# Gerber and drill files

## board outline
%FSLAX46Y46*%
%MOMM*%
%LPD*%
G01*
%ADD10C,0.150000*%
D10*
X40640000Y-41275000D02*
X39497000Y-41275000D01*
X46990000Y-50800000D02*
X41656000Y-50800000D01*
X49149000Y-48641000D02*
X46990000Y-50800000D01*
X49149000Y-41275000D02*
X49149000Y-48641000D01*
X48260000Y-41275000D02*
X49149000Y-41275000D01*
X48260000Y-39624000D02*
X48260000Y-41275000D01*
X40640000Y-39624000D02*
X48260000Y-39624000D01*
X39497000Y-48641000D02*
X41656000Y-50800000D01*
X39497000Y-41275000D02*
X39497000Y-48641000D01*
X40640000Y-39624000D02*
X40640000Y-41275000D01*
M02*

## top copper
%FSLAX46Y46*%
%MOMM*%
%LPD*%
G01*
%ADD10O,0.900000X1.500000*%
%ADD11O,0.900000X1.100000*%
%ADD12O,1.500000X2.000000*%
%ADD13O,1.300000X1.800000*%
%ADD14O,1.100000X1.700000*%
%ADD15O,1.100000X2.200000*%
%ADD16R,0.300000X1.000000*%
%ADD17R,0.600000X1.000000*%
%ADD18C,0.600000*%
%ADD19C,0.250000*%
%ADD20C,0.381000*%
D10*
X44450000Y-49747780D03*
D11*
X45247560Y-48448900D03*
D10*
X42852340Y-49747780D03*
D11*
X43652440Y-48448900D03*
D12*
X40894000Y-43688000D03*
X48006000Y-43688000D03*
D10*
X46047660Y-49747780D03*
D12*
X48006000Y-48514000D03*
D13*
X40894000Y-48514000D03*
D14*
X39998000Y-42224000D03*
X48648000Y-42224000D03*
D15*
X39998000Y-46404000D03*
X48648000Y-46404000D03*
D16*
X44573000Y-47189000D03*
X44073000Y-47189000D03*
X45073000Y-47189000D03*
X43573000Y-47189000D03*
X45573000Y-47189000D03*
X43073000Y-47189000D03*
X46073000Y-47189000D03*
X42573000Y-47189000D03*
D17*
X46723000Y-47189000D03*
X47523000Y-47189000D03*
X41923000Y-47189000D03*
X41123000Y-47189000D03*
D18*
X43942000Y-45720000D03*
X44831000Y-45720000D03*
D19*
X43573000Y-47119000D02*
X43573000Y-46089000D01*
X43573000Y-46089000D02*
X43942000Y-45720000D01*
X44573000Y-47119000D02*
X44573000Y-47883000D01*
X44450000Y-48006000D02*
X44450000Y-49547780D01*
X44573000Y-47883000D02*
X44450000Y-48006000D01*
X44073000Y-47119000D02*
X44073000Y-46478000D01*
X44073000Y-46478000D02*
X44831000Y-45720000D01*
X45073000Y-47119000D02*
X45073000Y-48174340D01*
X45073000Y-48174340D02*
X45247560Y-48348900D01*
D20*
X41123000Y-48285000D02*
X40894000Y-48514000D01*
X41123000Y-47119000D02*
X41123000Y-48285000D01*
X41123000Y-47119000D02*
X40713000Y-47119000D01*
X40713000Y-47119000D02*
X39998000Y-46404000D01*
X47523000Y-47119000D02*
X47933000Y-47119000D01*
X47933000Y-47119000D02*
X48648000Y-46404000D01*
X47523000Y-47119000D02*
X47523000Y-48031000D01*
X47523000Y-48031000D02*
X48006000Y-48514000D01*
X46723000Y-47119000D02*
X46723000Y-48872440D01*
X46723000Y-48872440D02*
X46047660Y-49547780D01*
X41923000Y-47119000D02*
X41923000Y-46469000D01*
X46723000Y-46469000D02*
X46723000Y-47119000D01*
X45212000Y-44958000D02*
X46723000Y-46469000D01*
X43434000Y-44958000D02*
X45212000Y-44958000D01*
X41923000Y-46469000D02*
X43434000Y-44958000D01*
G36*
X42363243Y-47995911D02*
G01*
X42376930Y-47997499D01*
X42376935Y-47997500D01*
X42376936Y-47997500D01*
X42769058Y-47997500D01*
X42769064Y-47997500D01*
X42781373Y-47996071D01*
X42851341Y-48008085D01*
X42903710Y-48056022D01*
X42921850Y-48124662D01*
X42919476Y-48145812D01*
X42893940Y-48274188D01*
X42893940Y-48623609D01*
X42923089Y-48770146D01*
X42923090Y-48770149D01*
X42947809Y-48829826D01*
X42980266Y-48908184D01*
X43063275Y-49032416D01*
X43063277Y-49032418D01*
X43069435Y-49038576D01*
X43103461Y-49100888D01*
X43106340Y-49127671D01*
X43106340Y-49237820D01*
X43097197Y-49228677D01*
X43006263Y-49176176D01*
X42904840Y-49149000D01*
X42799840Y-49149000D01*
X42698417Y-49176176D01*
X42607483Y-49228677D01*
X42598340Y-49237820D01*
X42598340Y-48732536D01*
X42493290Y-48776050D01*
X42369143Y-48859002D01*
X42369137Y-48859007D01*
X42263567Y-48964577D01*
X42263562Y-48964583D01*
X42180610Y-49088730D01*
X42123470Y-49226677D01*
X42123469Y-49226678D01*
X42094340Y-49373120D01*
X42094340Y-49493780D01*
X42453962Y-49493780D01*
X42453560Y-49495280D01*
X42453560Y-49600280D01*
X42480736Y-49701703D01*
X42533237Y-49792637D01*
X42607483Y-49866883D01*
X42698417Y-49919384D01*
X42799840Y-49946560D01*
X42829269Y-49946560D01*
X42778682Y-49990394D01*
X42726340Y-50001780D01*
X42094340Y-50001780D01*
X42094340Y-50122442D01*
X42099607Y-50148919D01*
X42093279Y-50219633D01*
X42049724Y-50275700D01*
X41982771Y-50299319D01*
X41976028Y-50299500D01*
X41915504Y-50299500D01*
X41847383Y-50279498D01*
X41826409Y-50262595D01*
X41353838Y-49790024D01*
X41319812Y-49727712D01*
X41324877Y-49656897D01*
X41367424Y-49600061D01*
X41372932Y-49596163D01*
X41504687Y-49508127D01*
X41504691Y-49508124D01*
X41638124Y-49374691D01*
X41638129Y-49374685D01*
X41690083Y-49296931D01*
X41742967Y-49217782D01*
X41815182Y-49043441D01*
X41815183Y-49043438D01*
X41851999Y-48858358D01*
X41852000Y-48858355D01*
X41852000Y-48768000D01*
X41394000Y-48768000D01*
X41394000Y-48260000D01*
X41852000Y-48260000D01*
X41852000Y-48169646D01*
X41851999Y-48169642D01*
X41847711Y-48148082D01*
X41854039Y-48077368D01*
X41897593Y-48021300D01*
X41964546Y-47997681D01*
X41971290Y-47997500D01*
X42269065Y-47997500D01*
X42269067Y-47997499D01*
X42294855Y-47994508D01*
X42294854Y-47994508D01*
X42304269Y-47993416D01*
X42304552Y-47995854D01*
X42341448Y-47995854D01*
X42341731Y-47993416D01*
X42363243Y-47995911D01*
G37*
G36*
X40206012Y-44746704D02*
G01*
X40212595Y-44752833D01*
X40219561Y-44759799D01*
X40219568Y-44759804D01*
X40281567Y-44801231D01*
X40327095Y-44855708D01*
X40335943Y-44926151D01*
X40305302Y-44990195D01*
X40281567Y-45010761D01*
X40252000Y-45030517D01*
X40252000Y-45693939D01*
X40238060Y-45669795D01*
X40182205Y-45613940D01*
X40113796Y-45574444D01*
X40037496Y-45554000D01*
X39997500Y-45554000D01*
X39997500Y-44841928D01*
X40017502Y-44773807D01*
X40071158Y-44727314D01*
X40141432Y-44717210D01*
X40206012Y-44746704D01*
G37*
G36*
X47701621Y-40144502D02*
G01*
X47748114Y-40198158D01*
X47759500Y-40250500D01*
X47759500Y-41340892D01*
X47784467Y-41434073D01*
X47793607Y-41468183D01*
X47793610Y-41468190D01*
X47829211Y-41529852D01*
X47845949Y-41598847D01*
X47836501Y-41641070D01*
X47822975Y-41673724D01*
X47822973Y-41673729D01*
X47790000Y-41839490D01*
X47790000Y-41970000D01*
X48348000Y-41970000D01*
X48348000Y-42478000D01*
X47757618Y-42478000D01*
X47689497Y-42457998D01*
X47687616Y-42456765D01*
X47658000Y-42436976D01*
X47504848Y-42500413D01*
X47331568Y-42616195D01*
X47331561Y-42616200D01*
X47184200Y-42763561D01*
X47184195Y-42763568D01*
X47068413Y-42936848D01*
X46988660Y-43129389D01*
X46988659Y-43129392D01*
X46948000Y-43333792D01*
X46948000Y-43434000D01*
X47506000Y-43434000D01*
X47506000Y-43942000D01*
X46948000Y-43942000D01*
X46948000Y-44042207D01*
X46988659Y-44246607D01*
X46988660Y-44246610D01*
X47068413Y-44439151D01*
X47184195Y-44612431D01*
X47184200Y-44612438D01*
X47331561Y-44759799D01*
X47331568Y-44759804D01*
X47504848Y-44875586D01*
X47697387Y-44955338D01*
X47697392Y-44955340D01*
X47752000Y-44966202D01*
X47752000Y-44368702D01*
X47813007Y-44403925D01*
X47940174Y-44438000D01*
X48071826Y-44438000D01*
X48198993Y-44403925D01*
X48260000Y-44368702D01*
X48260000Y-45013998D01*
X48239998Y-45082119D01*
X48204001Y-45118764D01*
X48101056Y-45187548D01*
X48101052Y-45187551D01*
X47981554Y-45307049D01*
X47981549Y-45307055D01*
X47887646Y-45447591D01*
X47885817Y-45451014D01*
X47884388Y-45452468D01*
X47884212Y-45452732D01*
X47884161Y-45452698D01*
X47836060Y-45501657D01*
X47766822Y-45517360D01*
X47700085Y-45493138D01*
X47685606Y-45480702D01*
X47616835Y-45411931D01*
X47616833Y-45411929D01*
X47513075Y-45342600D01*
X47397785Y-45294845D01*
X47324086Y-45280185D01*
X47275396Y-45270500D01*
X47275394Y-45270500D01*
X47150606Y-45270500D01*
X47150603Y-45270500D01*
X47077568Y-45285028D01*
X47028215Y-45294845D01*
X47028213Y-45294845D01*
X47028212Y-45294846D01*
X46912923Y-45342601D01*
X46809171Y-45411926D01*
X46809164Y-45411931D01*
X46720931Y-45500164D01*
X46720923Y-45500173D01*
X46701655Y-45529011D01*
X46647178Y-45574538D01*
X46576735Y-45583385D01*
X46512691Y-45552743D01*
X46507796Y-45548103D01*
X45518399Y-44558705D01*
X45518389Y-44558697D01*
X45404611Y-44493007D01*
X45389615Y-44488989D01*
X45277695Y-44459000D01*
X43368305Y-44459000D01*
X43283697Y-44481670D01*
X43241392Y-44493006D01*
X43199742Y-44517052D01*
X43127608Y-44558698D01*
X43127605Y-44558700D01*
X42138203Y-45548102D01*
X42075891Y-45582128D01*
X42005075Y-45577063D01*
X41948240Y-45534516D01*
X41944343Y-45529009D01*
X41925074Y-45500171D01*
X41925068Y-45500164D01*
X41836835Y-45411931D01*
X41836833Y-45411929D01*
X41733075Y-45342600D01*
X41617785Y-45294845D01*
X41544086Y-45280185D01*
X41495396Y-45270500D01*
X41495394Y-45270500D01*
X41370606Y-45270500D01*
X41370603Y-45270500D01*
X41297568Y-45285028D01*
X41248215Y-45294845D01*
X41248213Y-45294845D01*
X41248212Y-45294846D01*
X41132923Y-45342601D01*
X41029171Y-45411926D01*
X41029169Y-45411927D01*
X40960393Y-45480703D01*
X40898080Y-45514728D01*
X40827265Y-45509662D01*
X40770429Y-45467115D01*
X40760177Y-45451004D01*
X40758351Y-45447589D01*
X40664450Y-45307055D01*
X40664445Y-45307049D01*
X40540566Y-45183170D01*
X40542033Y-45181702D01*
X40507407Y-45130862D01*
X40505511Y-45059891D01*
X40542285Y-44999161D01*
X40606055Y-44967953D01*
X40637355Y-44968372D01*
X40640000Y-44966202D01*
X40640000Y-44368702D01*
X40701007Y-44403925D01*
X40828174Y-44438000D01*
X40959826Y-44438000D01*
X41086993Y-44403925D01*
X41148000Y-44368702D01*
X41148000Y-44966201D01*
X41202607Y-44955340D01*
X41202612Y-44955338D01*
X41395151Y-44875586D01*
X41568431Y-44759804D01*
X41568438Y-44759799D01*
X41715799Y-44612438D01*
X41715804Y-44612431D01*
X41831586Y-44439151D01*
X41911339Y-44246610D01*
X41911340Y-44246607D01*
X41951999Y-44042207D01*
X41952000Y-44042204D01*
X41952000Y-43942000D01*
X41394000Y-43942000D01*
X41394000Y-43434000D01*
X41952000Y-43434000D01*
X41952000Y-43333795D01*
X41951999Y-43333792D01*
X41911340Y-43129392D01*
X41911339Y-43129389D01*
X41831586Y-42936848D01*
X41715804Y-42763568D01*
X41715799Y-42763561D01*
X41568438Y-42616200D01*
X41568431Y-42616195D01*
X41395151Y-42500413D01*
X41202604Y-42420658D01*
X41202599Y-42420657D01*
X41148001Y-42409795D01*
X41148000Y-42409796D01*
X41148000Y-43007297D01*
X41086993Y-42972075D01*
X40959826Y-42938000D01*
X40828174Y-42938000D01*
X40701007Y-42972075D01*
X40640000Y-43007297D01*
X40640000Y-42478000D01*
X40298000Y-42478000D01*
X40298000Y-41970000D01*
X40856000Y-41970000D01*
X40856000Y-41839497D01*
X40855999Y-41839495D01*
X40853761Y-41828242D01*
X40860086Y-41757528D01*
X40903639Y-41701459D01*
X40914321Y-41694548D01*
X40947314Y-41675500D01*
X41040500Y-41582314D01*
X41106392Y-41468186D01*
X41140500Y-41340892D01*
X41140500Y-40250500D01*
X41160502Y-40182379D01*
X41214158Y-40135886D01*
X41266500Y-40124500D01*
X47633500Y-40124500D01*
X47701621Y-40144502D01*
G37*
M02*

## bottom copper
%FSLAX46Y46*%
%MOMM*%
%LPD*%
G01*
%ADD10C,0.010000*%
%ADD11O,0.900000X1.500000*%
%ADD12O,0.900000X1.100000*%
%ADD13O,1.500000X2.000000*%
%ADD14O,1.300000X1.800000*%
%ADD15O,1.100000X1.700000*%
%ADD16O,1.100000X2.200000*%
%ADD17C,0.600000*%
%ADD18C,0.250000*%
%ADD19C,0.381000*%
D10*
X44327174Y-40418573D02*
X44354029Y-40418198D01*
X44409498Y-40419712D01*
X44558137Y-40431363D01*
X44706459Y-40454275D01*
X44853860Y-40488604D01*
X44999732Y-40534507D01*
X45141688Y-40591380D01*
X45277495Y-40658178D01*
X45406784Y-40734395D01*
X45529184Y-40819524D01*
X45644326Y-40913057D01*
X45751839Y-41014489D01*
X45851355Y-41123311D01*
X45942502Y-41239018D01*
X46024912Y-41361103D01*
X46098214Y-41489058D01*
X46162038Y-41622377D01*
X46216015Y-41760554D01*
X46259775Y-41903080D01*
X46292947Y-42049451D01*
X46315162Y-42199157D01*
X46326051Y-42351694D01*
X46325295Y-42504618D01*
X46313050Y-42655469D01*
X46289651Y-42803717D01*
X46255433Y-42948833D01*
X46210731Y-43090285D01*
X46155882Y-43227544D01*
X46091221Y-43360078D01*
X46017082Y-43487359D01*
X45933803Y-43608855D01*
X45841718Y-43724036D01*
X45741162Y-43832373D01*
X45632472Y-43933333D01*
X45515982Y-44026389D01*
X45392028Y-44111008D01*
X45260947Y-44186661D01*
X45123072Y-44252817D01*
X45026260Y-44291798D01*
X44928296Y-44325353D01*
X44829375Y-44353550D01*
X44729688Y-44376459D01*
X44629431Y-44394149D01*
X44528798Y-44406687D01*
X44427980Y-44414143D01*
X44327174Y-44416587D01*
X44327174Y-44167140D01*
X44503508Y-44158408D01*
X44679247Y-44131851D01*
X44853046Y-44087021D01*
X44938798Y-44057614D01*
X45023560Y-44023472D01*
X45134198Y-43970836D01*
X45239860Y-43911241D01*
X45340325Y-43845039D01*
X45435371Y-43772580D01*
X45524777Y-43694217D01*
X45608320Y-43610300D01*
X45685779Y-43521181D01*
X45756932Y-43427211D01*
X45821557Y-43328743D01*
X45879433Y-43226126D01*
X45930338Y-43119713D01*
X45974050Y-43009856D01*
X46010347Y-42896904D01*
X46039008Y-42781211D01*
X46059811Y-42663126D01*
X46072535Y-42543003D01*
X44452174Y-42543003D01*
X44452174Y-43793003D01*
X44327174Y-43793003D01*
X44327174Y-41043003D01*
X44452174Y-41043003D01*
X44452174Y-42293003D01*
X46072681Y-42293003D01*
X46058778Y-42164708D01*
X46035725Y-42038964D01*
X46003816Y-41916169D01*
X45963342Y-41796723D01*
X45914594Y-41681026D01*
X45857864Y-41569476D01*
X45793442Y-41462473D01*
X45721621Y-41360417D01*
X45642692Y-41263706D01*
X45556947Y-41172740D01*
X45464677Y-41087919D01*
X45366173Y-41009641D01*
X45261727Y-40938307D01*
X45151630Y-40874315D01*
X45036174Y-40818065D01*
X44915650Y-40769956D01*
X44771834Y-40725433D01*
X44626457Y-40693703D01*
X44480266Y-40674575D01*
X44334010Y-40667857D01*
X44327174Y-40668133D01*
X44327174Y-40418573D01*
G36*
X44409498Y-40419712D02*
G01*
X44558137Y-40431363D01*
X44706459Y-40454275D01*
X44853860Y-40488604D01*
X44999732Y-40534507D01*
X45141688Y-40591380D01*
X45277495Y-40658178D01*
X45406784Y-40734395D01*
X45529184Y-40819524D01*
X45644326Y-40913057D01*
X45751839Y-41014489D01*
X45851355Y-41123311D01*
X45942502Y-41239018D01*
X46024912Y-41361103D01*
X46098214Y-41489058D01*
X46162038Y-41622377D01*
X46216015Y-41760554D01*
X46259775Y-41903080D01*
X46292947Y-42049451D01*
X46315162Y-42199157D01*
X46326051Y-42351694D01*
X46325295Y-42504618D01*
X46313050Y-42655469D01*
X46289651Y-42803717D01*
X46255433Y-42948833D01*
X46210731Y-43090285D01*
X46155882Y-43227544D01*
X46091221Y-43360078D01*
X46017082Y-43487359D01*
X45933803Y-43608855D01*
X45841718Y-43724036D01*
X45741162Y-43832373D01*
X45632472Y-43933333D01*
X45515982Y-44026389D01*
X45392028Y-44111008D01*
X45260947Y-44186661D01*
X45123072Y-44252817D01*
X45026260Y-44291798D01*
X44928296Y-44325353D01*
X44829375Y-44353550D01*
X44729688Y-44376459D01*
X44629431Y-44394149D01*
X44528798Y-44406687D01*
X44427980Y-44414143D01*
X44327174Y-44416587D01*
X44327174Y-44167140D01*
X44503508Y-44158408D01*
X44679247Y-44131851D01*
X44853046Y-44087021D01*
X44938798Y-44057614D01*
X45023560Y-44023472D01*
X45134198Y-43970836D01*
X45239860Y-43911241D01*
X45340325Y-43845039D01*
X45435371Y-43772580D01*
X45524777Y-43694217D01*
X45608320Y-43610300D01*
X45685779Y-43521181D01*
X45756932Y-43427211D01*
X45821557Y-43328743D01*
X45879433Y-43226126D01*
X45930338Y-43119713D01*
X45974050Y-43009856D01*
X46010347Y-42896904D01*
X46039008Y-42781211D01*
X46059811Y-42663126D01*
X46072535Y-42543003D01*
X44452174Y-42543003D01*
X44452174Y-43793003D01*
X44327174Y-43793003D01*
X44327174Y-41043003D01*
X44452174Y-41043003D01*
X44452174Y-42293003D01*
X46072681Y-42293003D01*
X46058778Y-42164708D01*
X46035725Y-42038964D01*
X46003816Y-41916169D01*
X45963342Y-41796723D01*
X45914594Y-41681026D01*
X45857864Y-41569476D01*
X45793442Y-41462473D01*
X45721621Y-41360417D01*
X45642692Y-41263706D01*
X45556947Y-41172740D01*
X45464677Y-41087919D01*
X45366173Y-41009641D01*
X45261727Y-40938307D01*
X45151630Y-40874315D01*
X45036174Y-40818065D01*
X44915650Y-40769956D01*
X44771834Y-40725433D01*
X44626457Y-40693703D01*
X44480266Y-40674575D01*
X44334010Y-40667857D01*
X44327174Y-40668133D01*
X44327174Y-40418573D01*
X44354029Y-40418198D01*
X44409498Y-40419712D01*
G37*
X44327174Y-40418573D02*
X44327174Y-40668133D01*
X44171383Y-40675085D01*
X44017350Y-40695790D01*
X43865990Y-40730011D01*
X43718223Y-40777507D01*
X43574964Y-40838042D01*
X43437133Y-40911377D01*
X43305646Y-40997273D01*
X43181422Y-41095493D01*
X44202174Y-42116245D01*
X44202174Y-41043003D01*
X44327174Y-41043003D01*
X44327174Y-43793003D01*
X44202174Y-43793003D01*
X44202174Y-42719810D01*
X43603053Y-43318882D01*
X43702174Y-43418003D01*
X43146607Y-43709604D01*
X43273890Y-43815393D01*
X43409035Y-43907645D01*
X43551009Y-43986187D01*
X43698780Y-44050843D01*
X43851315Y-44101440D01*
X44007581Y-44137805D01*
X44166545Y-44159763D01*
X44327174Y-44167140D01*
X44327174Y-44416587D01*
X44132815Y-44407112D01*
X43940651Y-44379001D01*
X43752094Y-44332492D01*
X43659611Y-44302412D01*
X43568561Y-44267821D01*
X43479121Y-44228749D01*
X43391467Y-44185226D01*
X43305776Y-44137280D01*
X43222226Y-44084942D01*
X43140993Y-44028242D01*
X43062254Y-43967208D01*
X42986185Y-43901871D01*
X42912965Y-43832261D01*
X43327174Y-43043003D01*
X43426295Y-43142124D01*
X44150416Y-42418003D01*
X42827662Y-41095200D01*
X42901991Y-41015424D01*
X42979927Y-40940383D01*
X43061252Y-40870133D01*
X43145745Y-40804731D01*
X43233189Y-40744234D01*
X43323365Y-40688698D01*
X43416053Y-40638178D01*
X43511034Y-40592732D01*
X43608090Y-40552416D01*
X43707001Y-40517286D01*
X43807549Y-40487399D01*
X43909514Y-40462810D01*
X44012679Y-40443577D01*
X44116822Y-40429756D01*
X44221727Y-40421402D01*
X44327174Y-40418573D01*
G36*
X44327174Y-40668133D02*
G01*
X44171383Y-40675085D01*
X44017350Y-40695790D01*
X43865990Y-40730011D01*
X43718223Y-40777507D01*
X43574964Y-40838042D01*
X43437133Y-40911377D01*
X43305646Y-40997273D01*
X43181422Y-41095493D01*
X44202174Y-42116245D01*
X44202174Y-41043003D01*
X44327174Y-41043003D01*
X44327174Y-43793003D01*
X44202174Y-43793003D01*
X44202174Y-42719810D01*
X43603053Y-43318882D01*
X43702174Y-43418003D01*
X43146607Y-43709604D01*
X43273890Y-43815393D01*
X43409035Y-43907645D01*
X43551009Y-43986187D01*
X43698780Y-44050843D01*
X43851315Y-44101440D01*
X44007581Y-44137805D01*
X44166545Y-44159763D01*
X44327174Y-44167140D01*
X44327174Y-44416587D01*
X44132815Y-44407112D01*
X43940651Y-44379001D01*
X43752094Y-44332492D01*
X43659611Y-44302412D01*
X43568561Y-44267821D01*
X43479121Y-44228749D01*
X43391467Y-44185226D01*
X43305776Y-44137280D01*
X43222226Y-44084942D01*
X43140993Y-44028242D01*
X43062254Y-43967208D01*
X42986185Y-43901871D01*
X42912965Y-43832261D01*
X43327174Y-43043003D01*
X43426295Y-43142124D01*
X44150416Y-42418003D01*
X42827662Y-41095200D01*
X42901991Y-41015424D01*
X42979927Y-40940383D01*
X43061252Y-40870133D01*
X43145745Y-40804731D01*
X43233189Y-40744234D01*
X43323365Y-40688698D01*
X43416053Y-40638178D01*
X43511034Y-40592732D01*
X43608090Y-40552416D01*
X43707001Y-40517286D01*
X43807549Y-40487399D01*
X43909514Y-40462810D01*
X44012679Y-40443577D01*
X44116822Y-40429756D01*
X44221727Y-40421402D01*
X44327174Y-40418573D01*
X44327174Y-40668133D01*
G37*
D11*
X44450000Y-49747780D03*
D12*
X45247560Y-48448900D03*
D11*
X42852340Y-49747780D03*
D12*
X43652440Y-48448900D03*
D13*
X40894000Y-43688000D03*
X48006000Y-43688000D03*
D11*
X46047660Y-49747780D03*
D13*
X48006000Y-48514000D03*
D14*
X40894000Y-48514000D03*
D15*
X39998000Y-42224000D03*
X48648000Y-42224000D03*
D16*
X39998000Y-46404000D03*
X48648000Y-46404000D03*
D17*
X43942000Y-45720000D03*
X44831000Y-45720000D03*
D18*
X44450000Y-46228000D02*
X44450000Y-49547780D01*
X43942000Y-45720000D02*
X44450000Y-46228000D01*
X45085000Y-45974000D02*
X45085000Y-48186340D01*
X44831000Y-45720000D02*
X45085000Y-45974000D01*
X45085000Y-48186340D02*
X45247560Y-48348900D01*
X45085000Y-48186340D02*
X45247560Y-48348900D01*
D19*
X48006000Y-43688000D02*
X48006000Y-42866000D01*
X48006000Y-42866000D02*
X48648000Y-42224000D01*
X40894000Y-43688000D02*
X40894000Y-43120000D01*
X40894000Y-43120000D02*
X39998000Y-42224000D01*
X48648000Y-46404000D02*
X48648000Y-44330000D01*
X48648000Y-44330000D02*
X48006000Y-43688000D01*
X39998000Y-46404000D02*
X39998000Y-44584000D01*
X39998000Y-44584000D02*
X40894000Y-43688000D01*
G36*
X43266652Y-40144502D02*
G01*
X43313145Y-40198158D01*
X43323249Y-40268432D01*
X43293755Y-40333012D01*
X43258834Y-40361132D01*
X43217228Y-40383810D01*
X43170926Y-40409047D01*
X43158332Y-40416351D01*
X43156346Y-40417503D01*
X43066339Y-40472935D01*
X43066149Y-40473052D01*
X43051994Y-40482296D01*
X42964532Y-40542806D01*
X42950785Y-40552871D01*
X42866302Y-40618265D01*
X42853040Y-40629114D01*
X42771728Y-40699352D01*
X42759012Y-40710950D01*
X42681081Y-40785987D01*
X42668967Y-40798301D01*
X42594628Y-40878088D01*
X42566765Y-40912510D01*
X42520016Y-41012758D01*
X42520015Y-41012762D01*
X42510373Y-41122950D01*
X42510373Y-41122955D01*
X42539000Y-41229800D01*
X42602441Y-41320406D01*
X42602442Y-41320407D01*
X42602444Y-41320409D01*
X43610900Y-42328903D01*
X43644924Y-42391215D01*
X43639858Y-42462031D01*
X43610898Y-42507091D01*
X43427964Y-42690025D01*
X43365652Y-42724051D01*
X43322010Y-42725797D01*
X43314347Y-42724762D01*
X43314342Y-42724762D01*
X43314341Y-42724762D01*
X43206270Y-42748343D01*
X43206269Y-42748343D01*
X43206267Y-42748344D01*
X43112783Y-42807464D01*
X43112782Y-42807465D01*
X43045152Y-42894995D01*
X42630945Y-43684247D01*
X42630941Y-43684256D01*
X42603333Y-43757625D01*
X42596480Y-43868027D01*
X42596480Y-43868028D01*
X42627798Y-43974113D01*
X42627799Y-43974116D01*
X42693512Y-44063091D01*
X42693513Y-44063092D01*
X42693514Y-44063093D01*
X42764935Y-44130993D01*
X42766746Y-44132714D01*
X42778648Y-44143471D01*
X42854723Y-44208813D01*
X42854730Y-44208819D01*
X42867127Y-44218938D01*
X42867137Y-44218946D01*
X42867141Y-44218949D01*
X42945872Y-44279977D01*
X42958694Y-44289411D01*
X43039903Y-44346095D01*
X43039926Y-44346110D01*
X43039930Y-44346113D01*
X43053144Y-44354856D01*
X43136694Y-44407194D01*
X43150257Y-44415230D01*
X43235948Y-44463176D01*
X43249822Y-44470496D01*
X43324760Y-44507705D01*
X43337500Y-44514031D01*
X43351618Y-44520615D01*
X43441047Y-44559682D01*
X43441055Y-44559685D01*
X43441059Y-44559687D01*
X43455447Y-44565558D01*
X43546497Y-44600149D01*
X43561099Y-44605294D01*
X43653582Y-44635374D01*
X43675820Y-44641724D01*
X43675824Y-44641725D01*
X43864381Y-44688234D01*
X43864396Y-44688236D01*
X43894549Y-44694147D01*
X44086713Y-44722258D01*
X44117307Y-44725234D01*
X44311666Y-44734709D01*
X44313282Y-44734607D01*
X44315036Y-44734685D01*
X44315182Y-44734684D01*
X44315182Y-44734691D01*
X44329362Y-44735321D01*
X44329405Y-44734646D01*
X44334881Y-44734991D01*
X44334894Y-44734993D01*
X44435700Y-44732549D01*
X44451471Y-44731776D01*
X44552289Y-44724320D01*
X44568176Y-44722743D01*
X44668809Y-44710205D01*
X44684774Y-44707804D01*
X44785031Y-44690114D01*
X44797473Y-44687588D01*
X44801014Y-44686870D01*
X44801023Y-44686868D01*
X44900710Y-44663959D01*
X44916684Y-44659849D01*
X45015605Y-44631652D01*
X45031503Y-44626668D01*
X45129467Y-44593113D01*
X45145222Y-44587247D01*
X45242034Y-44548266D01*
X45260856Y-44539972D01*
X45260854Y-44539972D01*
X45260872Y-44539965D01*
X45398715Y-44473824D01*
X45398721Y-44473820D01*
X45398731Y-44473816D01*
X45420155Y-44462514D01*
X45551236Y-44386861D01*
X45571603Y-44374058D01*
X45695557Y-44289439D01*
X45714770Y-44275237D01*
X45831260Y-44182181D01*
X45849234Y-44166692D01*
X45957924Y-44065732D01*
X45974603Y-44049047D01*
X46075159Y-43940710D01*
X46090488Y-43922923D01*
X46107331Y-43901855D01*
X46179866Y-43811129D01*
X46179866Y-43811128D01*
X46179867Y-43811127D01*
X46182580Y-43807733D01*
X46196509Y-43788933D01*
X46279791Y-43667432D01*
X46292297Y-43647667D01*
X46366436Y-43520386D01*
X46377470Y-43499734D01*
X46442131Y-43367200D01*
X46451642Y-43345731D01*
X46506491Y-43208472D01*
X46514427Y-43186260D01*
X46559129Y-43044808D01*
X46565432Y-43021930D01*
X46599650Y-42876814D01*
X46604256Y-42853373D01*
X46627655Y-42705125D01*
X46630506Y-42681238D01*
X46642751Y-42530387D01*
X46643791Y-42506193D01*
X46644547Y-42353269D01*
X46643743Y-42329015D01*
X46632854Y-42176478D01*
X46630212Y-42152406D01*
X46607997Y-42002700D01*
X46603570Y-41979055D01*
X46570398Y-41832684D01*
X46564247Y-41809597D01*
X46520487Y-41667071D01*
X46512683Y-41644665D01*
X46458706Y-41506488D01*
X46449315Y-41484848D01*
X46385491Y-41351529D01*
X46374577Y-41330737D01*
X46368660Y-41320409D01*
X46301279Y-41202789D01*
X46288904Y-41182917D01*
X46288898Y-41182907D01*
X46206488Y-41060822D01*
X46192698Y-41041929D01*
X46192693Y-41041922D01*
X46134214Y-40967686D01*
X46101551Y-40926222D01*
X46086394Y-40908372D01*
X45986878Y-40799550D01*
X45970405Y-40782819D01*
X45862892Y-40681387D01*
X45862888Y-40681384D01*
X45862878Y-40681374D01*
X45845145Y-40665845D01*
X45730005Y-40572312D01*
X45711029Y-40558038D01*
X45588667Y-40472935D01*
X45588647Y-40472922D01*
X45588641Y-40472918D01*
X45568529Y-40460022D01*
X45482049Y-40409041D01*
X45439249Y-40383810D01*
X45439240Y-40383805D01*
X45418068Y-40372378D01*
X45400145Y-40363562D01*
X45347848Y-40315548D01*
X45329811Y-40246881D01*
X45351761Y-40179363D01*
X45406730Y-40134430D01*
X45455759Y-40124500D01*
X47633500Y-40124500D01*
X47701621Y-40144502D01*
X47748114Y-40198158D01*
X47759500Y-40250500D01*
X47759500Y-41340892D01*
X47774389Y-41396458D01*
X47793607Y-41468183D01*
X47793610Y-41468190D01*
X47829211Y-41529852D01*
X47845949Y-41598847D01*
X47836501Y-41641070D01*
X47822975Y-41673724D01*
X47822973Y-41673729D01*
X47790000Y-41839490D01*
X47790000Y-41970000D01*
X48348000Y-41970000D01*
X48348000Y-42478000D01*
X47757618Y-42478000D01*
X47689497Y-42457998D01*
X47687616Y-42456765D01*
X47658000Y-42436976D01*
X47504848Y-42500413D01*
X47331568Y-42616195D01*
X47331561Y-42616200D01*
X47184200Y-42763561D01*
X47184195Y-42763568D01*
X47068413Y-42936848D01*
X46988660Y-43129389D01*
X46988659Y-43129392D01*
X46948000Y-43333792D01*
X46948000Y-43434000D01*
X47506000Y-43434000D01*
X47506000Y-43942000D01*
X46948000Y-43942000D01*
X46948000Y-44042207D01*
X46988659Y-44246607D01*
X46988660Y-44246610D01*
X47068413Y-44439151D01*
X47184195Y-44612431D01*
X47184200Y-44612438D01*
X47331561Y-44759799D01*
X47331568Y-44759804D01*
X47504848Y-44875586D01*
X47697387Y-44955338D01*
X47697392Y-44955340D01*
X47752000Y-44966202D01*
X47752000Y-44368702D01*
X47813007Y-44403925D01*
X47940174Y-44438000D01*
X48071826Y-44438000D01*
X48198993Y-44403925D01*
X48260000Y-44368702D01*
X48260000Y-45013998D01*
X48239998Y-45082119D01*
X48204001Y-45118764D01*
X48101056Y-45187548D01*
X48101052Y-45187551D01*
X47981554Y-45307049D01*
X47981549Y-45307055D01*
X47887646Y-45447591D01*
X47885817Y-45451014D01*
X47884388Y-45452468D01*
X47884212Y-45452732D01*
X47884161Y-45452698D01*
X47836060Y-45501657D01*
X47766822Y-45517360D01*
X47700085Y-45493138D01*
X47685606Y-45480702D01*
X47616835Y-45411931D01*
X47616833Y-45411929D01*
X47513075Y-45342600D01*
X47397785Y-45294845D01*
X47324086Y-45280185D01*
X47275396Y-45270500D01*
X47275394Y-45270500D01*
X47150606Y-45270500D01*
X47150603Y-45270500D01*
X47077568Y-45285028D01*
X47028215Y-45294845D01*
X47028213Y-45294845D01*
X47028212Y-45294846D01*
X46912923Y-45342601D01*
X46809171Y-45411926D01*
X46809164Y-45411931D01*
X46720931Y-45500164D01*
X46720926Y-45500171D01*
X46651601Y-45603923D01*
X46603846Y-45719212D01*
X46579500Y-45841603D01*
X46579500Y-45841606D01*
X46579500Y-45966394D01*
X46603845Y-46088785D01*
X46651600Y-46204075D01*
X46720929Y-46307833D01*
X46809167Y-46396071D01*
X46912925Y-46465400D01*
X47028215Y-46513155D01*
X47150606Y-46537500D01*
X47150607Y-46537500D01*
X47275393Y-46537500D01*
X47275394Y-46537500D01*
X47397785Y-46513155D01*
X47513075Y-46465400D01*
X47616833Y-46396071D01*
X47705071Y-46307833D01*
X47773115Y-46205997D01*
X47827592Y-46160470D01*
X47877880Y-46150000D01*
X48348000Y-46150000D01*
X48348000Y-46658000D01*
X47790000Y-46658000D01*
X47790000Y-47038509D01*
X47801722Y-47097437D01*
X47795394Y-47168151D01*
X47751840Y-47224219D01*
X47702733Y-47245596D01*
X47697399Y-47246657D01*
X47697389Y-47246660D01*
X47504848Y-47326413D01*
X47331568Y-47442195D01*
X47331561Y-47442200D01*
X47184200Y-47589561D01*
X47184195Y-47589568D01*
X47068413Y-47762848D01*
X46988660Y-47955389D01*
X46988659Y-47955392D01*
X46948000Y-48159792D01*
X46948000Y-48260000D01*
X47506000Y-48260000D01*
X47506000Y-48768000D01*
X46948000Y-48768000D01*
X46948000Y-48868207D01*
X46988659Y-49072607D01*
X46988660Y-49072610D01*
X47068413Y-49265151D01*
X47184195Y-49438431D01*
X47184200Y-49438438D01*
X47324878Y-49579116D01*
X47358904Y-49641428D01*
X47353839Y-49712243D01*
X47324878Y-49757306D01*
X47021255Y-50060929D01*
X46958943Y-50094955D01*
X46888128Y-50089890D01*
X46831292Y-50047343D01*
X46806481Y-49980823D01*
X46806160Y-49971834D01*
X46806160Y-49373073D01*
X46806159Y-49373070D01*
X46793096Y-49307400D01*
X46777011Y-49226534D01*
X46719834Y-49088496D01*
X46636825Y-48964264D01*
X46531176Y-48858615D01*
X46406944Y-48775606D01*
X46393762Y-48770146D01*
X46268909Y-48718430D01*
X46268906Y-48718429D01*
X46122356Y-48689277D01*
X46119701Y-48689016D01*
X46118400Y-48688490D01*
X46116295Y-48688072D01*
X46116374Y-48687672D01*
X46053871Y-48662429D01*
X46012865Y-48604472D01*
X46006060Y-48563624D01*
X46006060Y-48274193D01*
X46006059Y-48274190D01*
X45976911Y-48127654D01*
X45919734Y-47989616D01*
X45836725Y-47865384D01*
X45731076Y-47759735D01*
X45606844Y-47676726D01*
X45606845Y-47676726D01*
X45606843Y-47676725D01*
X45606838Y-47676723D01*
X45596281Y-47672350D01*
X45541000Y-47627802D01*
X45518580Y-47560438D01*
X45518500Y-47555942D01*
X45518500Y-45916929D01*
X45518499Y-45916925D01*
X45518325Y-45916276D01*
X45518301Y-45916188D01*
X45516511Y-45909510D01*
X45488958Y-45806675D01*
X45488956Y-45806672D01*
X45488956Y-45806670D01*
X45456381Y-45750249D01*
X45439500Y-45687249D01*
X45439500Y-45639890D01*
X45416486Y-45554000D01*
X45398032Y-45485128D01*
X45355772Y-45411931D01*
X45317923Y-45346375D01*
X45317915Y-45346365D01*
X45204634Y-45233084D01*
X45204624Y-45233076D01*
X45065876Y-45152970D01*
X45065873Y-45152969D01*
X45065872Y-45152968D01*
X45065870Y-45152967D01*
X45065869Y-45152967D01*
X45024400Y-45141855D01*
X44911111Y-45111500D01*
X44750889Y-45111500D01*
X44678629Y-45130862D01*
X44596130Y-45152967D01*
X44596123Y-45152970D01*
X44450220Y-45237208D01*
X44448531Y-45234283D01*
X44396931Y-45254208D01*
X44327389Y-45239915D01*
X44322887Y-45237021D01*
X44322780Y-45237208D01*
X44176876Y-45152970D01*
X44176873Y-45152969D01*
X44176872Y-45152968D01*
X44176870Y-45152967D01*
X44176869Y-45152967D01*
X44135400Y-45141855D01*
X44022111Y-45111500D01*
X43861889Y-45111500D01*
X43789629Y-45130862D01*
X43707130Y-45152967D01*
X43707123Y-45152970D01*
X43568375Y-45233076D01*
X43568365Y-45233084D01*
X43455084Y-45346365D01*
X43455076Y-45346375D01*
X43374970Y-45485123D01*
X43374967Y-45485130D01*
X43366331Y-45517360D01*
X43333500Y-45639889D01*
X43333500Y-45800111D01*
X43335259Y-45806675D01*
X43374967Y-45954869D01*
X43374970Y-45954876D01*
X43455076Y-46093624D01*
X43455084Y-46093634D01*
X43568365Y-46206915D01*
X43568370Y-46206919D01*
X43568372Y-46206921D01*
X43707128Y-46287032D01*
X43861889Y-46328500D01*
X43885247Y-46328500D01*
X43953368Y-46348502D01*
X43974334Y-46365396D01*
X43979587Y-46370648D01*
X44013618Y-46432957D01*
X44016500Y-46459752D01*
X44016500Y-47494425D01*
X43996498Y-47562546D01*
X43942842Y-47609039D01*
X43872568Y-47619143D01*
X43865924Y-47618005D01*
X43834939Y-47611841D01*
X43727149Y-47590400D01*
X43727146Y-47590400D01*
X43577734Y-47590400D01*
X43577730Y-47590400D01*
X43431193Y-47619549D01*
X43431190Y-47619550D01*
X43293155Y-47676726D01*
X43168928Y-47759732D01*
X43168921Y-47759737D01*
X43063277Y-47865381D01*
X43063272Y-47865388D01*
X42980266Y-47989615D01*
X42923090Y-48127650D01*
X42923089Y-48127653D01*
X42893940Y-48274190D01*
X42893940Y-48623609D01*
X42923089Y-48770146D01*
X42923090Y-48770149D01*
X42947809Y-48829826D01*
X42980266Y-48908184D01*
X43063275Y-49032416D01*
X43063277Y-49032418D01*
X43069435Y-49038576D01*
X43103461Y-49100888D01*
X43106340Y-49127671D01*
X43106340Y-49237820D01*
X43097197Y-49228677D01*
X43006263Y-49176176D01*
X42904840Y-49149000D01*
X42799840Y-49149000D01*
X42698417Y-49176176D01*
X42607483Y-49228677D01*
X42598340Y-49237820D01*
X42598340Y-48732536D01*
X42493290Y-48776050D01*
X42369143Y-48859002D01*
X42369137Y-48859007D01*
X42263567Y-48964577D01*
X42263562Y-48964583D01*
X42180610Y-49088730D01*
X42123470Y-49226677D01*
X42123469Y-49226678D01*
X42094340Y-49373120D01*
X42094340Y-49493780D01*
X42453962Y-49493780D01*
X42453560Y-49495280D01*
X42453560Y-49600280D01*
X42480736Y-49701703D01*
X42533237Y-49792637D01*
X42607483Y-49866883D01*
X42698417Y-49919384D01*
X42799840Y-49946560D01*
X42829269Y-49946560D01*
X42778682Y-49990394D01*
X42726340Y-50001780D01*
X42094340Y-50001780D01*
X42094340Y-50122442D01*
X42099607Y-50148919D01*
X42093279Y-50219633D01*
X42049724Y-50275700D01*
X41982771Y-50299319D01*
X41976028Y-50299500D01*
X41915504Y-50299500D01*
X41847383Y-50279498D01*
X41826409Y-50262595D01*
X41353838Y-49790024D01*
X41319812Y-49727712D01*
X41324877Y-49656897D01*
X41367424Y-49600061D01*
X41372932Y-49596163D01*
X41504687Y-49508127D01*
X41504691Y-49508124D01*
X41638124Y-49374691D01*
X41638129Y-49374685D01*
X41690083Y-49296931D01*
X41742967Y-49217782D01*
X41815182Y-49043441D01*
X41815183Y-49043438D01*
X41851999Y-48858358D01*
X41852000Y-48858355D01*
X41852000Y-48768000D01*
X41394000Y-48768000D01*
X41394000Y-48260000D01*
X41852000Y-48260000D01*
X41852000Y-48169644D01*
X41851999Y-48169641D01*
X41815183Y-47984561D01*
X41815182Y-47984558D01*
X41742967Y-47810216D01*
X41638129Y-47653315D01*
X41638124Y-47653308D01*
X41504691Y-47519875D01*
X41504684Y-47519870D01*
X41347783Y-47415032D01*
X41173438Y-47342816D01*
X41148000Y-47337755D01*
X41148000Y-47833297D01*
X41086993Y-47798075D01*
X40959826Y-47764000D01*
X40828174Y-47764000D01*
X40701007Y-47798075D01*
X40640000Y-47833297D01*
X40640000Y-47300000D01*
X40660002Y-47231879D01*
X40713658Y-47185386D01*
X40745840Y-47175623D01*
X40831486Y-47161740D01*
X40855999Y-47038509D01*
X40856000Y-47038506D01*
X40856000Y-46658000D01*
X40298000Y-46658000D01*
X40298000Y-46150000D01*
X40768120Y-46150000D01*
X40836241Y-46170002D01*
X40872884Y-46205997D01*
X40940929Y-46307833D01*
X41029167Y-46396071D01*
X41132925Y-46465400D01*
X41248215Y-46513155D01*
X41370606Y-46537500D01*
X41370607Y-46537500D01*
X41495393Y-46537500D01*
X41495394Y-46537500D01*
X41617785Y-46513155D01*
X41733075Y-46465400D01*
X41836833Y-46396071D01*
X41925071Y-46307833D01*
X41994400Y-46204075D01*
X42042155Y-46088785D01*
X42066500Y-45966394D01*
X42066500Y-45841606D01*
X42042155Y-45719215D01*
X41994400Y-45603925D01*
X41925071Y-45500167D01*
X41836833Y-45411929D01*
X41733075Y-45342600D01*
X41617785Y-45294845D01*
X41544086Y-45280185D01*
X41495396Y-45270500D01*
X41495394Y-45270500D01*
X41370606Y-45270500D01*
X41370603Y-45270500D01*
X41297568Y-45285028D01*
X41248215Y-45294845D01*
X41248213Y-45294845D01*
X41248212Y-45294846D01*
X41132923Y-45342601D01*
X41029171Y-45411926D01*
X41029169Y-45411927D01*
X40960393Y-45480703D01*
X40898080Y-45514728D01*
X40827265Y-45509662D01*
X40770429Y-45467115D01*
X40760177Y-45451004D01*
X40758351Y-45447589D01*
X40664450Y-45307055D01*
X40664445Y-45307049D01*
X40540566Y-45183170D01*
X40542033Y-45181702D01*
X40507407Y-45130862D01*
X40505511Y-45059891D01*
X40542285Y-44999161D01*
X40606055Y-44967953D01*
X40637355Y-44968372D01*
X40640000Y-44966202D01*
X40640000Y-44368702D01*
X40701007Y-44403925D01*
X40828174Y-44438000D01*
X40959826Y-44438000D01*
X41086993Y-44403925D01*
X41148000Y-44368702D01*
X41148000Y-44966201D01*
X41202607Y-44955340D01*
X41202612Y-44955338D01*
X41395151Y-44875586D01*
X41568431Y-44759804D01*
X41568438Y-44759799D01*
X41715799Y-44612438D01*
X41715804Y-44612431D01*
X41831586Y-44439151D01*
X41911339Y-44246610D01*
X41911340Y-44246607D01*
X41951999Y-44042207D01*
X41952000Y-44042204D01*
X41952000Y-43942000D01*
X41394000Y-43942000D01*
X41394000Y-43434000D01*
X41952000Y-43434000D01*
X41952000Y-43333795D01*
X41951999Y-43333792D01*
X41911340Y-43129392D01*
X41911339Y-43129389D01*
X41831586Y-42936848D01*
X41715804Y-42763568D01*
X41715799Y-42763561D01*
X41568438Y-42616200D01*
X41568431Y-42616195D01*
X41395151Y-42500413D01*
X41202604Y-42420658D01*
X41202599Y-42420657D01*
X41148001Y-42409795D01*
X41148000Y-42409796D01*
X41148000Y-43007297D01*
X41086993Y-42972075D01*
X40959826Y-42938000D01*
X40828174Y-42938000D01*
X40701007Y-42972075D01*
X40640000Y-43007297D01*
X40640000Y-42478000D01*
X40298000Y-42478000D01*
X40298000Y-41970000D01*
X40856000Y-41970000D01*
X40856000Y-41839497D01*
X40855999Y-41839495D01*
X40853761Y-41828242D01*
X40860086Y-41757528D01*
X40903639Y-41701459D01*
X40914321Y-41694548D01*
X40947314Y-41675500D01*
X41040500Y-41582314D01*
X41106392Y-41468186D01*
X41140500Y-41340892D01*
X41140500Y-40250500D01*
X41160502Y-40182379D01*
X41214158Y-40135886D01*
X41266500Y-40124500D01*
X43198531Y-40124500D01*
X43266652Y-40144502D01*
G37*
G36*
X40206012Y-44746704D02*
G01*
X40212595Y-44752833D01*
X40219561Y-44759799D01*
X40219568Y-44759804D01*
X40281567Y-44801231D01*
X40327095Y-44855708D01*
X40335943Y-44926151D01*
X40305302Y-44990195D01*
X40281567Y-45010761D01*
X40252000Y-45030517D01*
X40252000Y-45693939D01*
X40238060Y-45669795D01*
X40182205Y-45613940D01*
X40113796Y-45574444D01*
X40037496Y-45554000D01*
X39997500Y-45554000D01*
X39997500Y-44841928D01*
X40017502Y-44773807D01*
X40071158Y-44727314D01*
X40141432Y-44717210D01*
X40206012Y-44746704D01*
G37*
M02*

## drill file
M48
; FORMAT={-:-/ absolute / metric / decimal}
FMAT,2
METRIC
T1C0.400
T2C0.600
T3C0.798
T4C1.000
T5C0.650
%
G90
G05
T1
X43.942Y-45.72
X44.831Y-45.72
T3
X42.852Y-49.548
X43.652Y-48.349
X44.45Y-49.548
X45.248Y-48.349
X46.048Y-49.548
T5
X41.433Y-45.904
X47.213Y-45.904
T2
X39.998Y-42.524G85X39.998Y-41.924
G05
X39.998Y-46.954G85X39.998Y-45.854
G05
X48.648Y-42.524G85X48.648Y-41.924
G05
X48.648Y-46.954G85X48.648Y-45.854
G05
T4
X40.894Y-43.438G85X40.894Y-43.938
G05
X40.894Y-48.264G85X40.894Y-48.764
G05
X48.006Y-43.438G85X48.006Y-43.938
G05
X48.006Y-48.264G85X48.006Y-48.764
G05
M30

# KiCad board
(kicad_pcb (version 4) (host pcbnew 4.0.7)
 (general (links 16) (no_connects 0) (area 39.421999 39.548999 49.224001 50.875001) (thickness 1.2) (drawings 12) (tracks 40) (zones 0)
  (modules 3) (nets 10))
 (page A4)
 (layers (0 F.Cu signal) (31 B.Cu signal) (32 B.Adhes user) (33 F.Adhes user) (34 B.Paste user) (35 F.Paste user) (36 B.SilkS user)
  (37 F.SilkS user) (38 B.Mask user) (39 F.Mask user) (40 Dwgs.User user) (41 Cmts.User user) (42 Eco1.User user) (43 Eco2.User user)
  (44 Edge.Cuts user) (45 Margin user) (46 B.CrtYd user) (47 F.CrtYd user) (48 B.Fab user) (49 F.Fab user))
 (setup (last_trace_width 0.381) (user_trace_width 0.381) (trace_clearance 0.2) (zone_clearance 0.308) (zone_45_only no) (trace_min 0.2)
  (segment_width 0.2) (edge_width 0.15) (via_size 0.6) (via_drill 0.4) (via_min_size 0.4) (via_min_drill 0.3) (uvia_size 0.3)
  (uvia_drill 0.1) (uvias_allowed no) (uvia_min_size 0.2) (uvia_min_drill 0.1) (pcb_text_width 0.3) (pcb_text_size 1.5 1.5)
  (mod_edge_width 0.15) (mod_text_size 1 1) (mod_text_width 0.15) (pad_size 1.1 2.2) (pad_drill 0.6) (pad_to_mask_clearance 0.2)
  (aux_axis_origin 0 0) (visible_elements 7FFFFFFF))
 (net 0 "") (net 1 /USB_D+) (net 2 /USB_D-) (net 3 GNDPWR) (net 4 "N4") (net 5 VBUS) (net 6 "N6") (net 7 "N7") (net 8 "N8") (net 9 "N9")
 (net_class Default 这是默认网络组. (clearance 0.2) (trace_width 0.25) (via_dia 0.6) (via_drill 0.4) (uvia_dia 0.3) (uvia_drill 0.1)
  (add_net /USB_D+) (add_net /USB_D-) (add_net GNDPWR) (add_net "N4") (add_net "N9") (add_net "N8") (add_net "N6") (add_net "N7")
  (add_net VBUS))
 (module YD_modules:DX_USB (layer F.Cu) (at 44.45 44.45 270)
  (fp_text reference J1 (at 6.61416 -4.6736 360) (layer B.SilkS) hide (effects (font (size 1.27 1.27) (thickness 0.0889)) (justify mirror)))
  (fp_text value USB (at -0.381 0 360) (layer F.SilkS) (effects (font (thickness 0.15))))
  (pad 3 thru_hole oval (at 5.09778 0 270) (size 1.5 0.9) (drill 0.79756 (offset 0.2 0)) (layers *.Cu *.Paste *.Mask) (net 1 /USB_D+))
  (pad 2 thru_hole oval (at 3.8989 -0.79756 270) (size 1.1 0.9) (drill 0.79756 (offset 0.1 0)) (layers *.Cu *.Paste *.Mask) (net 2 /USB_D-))
  (pad 5 thru_hole oval (at 5.09778 1.59766 270) (size 1.5 0.9) (drill 0.79756 (offset 0.2 0)) (layers *.Cu *.Paste *.Mask) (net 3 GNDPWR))
  (pad 4 thru_hole oval (at 3.8989 0.79756 270) (size 1.1 0.9) (drill 0.79756 (offset 0.1 0)) (layers *.Cu *.Paste *.Mask) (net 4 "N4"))
  (pad P$6 thru_hole oval (at -0.762 3.556 270) (size 2 1.5) (drill oval 1.5 1) (layers *.Cu *.Mask F.Paste F.SilkS) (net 3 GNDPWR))
  (pad P$7 thru_hole oval (at -0.762 -3.556 270) (size 2 1.5) (drill oval 1.5 1) (layers *.Cu *.Mask F.Paste F.SilkS) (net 3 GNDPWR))
  (pad 1 thru_hole oval (at 5.09778 -1.59766 270) (size 1.5 0.9) (drill 0.79756 (offset 0.2 0)) (layers *.Cu *.Paste *.Mask) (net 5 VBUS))
  (pad P$8 thru_hole oval (at 4.064 -3.556 270) (size 2 1.5) (drill oval 1.5 1) (layers *.Cu *.Mask F.Paste F.SilkS) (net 3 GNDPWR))
  (pad P$9 thru_hole oval (at 4.064 3.556 270) (size 1.8 1.3) (drill oval 1.5 1) (layers *.Cu *.Mask F.Paste F.SilkS) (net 3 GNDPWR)))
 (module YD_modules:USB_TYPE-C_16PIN (layer F.Cu) (at 44.323 39.624 180)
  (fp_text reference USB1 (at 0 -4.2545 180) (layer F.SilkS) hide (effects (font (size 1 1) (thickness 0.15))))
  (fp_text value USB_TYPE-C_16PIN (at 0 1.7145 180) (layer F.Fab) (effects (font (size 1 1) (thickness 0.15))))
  (pad 0 thru_hole oval (at 4.325 -2.6 180) (size 1.1 1.7) (drill oval 0.6 1.2) (layers *.Cu *.Mask) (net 3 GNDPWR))
  (pad 0 thru_hole oval (at -4.325 -2.6 180) (size 1.1 1.7) (drill oval 0.6 1.2) (layers *.Cu *.Mask) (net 3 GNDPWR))
  (pad 0 thru_hole oval (at 4.325 -6.78 180) (size 1.1 2.2) (drill oval 0.6 1.7) (layers *.Cu *.Mask) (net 3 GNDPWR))
  (pad 0 thru_hole oval (at -4.325 -6.78 180) (size 1.1 2.2) (drill oval 0.6 1.7) (layers *.Cu *.Mask) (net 3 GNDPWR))
  (pad "" np_thru_hole oval (at 2.89 -6.28 180) (size 0.65 0.65) (drill 0.65) (layers *.Cu))
  (pad "" np_thru_hole oval (at -2.89 -6.28 180) (size 0.65 0.65) (drill 0.65) (layers *.Cu))
  (pad 6 smd rect (at -0.25 -7.495 180) (size 0.3 1) (drill (offset 0 -0.07)) (layers F.Cu F.Paste F.Mask) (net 1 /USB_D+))
  (pad 7 smd rect (at 0.25 -7.495 180) (size 0.3 1) (drill (offset 0 -0.07)) (layers F.Cu F.Paste F.Mask) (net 2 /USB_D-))
  (pad 5 smd rect (at -0.75 -7.495 180) (size 0.3 1) (drill (offset 0 -0.07)) (layers F.Cu F.Paste F.Mask) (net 2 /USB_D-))
  (pad 8 smd rect (at 0.75 -7.495 180) (size 0.3 1) (drill (offset 0 -0.07)) (layers F.Cu F.Paste F.Mask) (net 1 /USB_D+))
  (pad 4 smd rect (at -1.25 -7.495 180) (size 0.3 1) (drill (offset 0 -0.07)) (layers F.Cu F.Paste F.Mask) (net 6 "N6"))
  (pad 9 smd rect (at 1.25 -7.495 180) (size 0.3 1) (drill (offset 0 -0.07)) (layers F.Cu F.Paste F.Mask) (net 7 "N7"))
  (pad 3 smd rect (at -1.75 -7.495 180) (size 0.3 1) (drill (offset 0 -0.07)) (layers F.Cu F.Paste F.Mask) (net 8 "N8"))
  (pad 10 smd rect (at 1.75 -7.495 180) (size 0.3 1) (drill (offset 0 -0.07)) (layers F.Cu F.Paste F.Mask) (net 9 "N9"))
  (pad 2 smd rect (at -2.4 -7.495 180) (size 0.6 1) (drill (offset 0 -0.07)) (layers F.Cu F.Paste F.Mask) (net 5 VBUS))
  (pad 1 smd rect (at -3.2 -7.495 180) (size 0.6 1) (drill (offset 0 -0.07)) (layers F.Cu F.Paste F.Mask) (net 3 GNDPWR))
  (pad 11 smd rect (at 2.4 -7.495 180) (size 0.6 1) (drill (offset 0 -0.07)) (layers F.Cu F.Paste F.Mask) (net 5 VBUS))
  (pad 12 smd rect (at 3.2 -7.495 180) (size 0.6 1) (drill (offset 0 -0.07)) (layers F.Cu F.Paste F.Mask) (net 3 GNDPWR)))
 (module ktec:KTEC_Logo (layer B.Cu) (at 44.323 42.418 180)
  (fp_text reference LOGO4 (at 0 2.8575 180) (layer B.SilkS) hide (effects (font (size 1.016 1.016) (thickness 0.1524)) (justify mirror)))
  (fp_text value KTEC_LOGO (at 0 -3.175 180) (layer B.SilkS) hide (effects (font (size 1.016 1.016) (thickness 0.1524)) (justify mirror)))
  (fp_poly
   (pts (xy -0.004174 1.999427) (xy -0.031029 1.999802) (xy -0.086498 1.998288) (xy -0.235137 1.986637) (xy -0.383459 1.963725)
    (xy -0.53086 1.929396) (xy -0.676732 1.883493) (xy -0.818688 1.82662) (xy -0.954495 1.759822) (xy -1.083784 1.683605)
    (xy -1.206184 1.598476) (xy -1.321326 1.504943) (xy -1.428839 1.403511) (xy -1.528355 1.294689) (xy -1.619502 1.178982)
    (xy -1.701912 1.056897) (xy -1.775214 0.928942) (xy -1.839038 0.795623) (xy -1.893015 0.657446) (xy -1.936775 0.51492)
    (xy -1.969947 0.368549) (xy -1.992162 0.218843) (xy -2.003051 0.066306) (xy -2.002295 -0.086618) (xy -1.99005 -0.237469)
    (xy -1.966651 -0.385717) (xy -1.932433 -0.530833) (xy -1.887731 -0.672285) (xy -1.832882 -0.809544) (xy -1.768221 -0.942078)
    (xy -1.694082 -1.069359) (xy -1.610803 -1.190855) (xy -1.518718 -1.306036) (xy -1.418162 -1.414373) (xy -1.309472 -1.515333)
    (xy -1.192982 -1.608389) (xy -1.069028 -1.693008) (xy -0.937947 -1.768661) (xy -0.800072 -1.834817) (xy -0.70326 -1.873798)
    (xy -0.605296 -1.907353) (xy -0.506375 -1.93555) (xy -0.406688 -1.958459) (xy -0.306431 -1.976149) (xy -0.205798 -1.988687)
    (xy -0.10498 -1.996143) (xy -0.004174 -1.998587) (xy -0.004174 -1.74914) (xy -0.180508 -1.740408) (xy -0.356247 -1.713851)
    (xy -0.530046 -1.669021) (xy -0.615798 -1.639614) (xy -0.70056 -1.605472) (xy -0.811198 -1.552836) (xy -0.91686 -1.493241)
    (xy -1.017325 -1.427039) (xy -1.112371 -1.35458) (xy -1.201777 -1.276217) (xy -1.28532 -1.1923) (xy -1.362779 -1.103181)
    (xy -1.433932 -1.009211) (xy -1.498557 -0.910743) (xy -1.556433 -0.808126) (xy -1.607338 -0.701713) (xy -1.65105 -0.591856)
    (xy -1.687347 -0.478904) (xy -1.716008 -0.363211) (xy -1.736811 -0.245126) (xy -1.749535 -0.125003) (xy -0.129174 -0.125003)
    (xy -0.129174 -1.375003) (xy -0.004174 -1.375003) (xy -0.004174 1.374997) (xy -0.129174 1.374997) (xy -0.129174 0.124997)
    (xy -1.749681 0.124997) (xy -1.735778 0.253292) (xy -1.712725 0.379036) (xy -1.680816 0.501831) (xy -1.640342 0.621277)
    (xy -1.591594 0.736974) (xy -1.534864 0.848524) (xy -1.470442 0.955527) (xy -1.398621 1.057583) (xy -1.319692 1.154294)
    (xy -1.233947 1.24526) (xy -1.141677 1.330081) (xy -1.043173 1.408359) (xy -0.938727 1.479693) (xy -0.82863 1.543685)
    (xy -0.713174 1.599935) (xy -0.59265 1.648044) (xy -0.448834 1.692567) (xy -0.303457 1.724297) (xy -0.157266 1.743425)
    (xy -0.01101 1.750143) (xy -0.004174 1.749867) (xy -0.004174 1.999427) (xy -0.004174 1.999427))
   (layer B.Cu) (width 0.01))
  (fp_poly
   (pts (xy -0.004174 1.999427) (xy -0.004174 1.749867) (xy 0.151617 1.742915) (xy 0.30565 1.72221) (xy 0.45701 1.687989)
    (xy 0.604777 1.640493) (xy 0.748036 1.579958) (xy 0.885867 1.506623) (xy 1.017354 1.420727) (xy 1.141578 1.322507)
    (xy 0.120826 0.301755) (xy 0.120826 1.374997) (xy -0.004174 1.374997) (xy -0.004174 -1.375003) (xy 0.120826 -1.375003)
    (xy 0.120826 -0.30181) (xy 0.719947 -0.900882) (xy 0.620826 -1.000003) (xy 1.176393 -1.291604) (xy 1.04911 -1.397393)
    (xy 0.913965 -1.489645) (xy 0.771991 -1.568187) (xy 0.62422 -1.632843) (xy 0.471685 -1.68344) (xy 0.315419 -1.719805)
    (xy 0.156455 -1.741763) (xy -0.004174 -1.74914) (xy -0.004174 -1.998587) (xy 0.190185 -1.989112) (xy 0.382349 -1.961001)
    (xy 0.570906 -1.914492) (xy 0.663389 -1.884412) (xy 0.754439 -1.849821) (xy 0.843879 -1.810749) (xy 0.931533 -1.767226)
    (xy 1.017224 -1.71928) (xy 1.100774 -1.666942) (xy 1.182007 -1.610242) (xy 1.260746 -1.549208) (xy 1.336815 -1.483871)
    (xy 1.410035 -1.414261) (xy 0.995826 -0.625003) (xy 0.896705 -0.724124) (xy 0.172584 -0.000003) (xy 1.495338 1.3228)
    (xy 1.421009 1.402576) (xy 1.343073 1.477617) (xy 1.261748 1.547867) (xy 1.177255 1.613269) (xy 1.089811 1.673766)
    (xy 0.999635 1.729302) (xy 0.906947 1.779822) (xy 0.811966 1.825268) (xy 0.71491 1.865584) (xy 0.615999 1.900714) (xy 0.515451 1.930601)
    (xy 0.413486 1.95519) (xy 0.310321 1.974423) (xy 0.206178 1.988244) (xy 0.101273 1.996598) (xy -0.004174 1.999427)
    (xy -0.004174 1.999427))
   (layer B.Cu) (width 0.01)))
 (gr_line (start 40.64 41.275) (end 39.497 41.275) (angle 90) (layer Edge.Cuts) (width 0.15))
 (gr_line (start 46.99 50.8) (end 41.656 50.8) (angle 90) (layer Edge.Cuts) (width 0.15))
 (gr_line (start 49.149 48.641) (end 46.99 50.8) (angle 90) (layer Edge.Cuts) (width 0.15))
 (gr_line (start 49.149 41.275) (end 49.149 48.641) (angle 90) (layer Edge.Cuts) (width 0.15))
 (gr_line (start 48.26 41.275) (end 49.149 41.275) (angle 90) (layer Edge.Cuts) (width 0.15))
 (gr_line (start 48.26 39.624) (end 48.26 41.275) (angle 90) (layer Edge.Cuts) (width 0.15))
 (gr_line (start 40.64 39.624) (end 48.26 39.624) (angle 90) (layer Edge.Cuts) (width 0.15))
 (gr_line (start 39.497 48.641) (end 41.656 50.8) (angle 90) (layer Edge.Cuts) (width 0.15))
 (gr_line (start 39.497 41.275) (end 39.497 48.641) (angle 90) (layer Edge.Cuts) (width 0.15))
 (gr_line (start 40.64 39.624) (end 40.64 41.275) (angle 90) (layer Edge.Cuts) (width 0.15))
 (segment (start 43.573 47.119) (end 43.573 46.089) (width 0.25) (layer F.Cu) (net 1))
 (segment (start 44.45 46.228) (end 44.45 49.54778) (width 0.25) (layer B.Cu) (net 1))
 (segment (start 43.942 45.72) (end 44.45 46.228) (width 0.25) (layer B.Cu) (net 1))
 (via (at 43.942 45.72) (size 0.6) (drill 0.4) (layers F.Cu B.Cu) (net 1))
 (segment (start 43.573 46.089) (end 43.942 45.72) (width 0.25) (layer F.Cu) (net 1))
 (segment (start 44.573 47.119) (end 44.573 47.883) (width 0.25) (layer F.Cu) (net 1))
 (segment (start 44.45 48.006) (end 44.45 49.54778) (width 0.25) (layer F.Cu) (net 1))
 (segment (start 44.573 47.883) (end 44.45 48.006) (width 0.25) (layer F.Cu) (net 1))
 (segment (start 44.073 47.119) (end 44.073 46.478) (width 0.25) (layer F.Cu) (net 2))
 (segment (start 45.085 45.974) (end 45.085 48.18634) (width 0.25) (layer B.Cu) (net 2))
 (segment (start 44.831 45.72) (end 45.085 45.974) (width 0.25) (layer B.Cu) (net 2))
 (via (at 44.831 45.72) (size 0.6) (drill 0.4) (layers F.Cu B.Cu) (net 2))
 (segment (start 44.073 46.478) (end 44.831 45.72) (width 0.25) (layer F.Cu) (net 2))
 (segment (start 45.085 48.18634) (end 45.24756 48.3489) (width 0.25) (layer B.Cu) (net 2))
 (segment (start 45.085 48.18634) (end 45.24756 48.3489) (width 0.25) (layer B.Cu) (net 2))
 (segment (start 45.073 47.119) (end 45.073 48.17434) (width 0.25) (layer F.Cu) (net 2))
 (segment (start 45.073 48.17434) (end 45.24756 48.3489) (width 0.25) (layer F.Cu) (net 2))
 (segment (start 41.123 48.285) (end 40.894 48.514) (width 0.381) (layer F.Cu) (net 3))
 (segment (start 41.123 47.119) (end 41.123 48.285) (width 0.381) (layer F.Cu) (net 3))
 (segment (start 41.123 47.119) (end 40.713 47.119) (width 0.381) (layer F.Cu) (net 3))
 (segment (start 40.713 47.119) (end 39.998 46.404) (width 0.381) (layer F.Cu) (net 3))
 (segment (start 47.523 47.119) (end 47.933 47.119) (width 0.381) (layer F.Cu) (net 3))
 (segment (start 47.933 47.119) (end 48.648 46.404) (width 0.381) (layer F.Cu) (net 3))
 (segment (start 47.523 47.119) (end 47.523 48.031) (width 0.381) (layer F.Cu) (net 3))
 (segment (start 47.523 48.031) (end 48.006 48.514) (width 0.381) (layer F.Cu) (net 3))
 (segment (start 48.006 43.688) (end 48.006 42.866) (width 0.381) (layer B.Cu) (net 3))
 (segment (start 48.006 42.866) (end 48.648 42.224) (width 0.381) (layer B.Cu) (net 3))
 (segment (start 40.894 43.688) (end 40.894 43.12) (width 0.381) (layer B.Cu) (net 3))
 (segment (start 40.894 43.12) (end 39.998 42.224) (width 0.381) (layer B.Cu) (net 3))
 (segment (start 48.648 46.404) (end 48.648 44.33) (width 0.381) (layer B.Cu) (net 3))
 (segment (start 48.648 44.33) (end 48.006 43.688) (width 0.381) (layer B.Cu) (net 3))
 (segment (start 39.998 46.404) (end 39.998 44.584) (width 0.381) (layer B.Cu) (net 3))
 (segment (start 39.998 44.584) (end 40.894 43.688) (width 0.381) (layer B.Cu) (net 3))
 (segment (start 46.723 47.119) (end 46.723 48.87244) (width 0.381) (layer F.Cu) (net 5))
 (segment (start 46.723 48.87244) (end 46.04766 49.54778) (width 0.381) (layer F.Cu) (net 5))
 (segment (start 41.923 47.119) (end 41.923 46.469) (width 0.381) (layer F.Cu) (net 5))
 (segment (start 46.723 46.469) (end 46.723 47.119) (width 0.381) (layer F.Cu) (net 5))
 (segment (start 45.212 44.958) (end 46.723 46.469) (width 0.381) (layer F.Cu) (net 5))
 (segment (start 43.434 44.958) (end 45.212 44.958) (width 0.381) (layer F.Cu) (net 5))
 (segment (start 41.923 46.469) (end 43.434 44.958) (width 0.381) (layer F.Cu) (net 5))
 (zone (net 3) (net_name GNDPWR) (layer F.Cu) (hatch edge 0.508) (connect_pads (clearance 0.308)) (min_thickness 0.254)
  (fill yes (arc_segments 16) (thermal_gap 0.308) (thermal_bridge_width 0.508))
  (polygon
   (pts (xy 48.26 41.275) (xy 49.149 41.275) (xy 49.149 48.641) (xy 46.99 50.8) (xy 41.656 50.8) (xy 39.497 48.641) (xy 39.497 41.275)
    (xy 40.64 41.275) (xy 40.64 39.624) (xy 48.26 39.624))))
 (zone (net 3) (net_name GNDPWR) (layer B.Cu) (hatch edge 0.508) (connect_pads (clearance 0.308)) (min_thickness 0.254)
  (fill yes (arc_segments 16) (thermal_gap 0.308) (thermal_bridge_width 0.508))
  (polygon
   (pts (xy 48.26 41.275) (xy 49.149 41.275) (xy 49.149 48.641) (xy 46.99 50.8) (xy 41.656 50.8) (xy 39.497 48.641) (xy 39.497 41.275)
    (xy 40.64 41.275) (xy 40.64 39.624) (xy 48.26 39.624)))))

